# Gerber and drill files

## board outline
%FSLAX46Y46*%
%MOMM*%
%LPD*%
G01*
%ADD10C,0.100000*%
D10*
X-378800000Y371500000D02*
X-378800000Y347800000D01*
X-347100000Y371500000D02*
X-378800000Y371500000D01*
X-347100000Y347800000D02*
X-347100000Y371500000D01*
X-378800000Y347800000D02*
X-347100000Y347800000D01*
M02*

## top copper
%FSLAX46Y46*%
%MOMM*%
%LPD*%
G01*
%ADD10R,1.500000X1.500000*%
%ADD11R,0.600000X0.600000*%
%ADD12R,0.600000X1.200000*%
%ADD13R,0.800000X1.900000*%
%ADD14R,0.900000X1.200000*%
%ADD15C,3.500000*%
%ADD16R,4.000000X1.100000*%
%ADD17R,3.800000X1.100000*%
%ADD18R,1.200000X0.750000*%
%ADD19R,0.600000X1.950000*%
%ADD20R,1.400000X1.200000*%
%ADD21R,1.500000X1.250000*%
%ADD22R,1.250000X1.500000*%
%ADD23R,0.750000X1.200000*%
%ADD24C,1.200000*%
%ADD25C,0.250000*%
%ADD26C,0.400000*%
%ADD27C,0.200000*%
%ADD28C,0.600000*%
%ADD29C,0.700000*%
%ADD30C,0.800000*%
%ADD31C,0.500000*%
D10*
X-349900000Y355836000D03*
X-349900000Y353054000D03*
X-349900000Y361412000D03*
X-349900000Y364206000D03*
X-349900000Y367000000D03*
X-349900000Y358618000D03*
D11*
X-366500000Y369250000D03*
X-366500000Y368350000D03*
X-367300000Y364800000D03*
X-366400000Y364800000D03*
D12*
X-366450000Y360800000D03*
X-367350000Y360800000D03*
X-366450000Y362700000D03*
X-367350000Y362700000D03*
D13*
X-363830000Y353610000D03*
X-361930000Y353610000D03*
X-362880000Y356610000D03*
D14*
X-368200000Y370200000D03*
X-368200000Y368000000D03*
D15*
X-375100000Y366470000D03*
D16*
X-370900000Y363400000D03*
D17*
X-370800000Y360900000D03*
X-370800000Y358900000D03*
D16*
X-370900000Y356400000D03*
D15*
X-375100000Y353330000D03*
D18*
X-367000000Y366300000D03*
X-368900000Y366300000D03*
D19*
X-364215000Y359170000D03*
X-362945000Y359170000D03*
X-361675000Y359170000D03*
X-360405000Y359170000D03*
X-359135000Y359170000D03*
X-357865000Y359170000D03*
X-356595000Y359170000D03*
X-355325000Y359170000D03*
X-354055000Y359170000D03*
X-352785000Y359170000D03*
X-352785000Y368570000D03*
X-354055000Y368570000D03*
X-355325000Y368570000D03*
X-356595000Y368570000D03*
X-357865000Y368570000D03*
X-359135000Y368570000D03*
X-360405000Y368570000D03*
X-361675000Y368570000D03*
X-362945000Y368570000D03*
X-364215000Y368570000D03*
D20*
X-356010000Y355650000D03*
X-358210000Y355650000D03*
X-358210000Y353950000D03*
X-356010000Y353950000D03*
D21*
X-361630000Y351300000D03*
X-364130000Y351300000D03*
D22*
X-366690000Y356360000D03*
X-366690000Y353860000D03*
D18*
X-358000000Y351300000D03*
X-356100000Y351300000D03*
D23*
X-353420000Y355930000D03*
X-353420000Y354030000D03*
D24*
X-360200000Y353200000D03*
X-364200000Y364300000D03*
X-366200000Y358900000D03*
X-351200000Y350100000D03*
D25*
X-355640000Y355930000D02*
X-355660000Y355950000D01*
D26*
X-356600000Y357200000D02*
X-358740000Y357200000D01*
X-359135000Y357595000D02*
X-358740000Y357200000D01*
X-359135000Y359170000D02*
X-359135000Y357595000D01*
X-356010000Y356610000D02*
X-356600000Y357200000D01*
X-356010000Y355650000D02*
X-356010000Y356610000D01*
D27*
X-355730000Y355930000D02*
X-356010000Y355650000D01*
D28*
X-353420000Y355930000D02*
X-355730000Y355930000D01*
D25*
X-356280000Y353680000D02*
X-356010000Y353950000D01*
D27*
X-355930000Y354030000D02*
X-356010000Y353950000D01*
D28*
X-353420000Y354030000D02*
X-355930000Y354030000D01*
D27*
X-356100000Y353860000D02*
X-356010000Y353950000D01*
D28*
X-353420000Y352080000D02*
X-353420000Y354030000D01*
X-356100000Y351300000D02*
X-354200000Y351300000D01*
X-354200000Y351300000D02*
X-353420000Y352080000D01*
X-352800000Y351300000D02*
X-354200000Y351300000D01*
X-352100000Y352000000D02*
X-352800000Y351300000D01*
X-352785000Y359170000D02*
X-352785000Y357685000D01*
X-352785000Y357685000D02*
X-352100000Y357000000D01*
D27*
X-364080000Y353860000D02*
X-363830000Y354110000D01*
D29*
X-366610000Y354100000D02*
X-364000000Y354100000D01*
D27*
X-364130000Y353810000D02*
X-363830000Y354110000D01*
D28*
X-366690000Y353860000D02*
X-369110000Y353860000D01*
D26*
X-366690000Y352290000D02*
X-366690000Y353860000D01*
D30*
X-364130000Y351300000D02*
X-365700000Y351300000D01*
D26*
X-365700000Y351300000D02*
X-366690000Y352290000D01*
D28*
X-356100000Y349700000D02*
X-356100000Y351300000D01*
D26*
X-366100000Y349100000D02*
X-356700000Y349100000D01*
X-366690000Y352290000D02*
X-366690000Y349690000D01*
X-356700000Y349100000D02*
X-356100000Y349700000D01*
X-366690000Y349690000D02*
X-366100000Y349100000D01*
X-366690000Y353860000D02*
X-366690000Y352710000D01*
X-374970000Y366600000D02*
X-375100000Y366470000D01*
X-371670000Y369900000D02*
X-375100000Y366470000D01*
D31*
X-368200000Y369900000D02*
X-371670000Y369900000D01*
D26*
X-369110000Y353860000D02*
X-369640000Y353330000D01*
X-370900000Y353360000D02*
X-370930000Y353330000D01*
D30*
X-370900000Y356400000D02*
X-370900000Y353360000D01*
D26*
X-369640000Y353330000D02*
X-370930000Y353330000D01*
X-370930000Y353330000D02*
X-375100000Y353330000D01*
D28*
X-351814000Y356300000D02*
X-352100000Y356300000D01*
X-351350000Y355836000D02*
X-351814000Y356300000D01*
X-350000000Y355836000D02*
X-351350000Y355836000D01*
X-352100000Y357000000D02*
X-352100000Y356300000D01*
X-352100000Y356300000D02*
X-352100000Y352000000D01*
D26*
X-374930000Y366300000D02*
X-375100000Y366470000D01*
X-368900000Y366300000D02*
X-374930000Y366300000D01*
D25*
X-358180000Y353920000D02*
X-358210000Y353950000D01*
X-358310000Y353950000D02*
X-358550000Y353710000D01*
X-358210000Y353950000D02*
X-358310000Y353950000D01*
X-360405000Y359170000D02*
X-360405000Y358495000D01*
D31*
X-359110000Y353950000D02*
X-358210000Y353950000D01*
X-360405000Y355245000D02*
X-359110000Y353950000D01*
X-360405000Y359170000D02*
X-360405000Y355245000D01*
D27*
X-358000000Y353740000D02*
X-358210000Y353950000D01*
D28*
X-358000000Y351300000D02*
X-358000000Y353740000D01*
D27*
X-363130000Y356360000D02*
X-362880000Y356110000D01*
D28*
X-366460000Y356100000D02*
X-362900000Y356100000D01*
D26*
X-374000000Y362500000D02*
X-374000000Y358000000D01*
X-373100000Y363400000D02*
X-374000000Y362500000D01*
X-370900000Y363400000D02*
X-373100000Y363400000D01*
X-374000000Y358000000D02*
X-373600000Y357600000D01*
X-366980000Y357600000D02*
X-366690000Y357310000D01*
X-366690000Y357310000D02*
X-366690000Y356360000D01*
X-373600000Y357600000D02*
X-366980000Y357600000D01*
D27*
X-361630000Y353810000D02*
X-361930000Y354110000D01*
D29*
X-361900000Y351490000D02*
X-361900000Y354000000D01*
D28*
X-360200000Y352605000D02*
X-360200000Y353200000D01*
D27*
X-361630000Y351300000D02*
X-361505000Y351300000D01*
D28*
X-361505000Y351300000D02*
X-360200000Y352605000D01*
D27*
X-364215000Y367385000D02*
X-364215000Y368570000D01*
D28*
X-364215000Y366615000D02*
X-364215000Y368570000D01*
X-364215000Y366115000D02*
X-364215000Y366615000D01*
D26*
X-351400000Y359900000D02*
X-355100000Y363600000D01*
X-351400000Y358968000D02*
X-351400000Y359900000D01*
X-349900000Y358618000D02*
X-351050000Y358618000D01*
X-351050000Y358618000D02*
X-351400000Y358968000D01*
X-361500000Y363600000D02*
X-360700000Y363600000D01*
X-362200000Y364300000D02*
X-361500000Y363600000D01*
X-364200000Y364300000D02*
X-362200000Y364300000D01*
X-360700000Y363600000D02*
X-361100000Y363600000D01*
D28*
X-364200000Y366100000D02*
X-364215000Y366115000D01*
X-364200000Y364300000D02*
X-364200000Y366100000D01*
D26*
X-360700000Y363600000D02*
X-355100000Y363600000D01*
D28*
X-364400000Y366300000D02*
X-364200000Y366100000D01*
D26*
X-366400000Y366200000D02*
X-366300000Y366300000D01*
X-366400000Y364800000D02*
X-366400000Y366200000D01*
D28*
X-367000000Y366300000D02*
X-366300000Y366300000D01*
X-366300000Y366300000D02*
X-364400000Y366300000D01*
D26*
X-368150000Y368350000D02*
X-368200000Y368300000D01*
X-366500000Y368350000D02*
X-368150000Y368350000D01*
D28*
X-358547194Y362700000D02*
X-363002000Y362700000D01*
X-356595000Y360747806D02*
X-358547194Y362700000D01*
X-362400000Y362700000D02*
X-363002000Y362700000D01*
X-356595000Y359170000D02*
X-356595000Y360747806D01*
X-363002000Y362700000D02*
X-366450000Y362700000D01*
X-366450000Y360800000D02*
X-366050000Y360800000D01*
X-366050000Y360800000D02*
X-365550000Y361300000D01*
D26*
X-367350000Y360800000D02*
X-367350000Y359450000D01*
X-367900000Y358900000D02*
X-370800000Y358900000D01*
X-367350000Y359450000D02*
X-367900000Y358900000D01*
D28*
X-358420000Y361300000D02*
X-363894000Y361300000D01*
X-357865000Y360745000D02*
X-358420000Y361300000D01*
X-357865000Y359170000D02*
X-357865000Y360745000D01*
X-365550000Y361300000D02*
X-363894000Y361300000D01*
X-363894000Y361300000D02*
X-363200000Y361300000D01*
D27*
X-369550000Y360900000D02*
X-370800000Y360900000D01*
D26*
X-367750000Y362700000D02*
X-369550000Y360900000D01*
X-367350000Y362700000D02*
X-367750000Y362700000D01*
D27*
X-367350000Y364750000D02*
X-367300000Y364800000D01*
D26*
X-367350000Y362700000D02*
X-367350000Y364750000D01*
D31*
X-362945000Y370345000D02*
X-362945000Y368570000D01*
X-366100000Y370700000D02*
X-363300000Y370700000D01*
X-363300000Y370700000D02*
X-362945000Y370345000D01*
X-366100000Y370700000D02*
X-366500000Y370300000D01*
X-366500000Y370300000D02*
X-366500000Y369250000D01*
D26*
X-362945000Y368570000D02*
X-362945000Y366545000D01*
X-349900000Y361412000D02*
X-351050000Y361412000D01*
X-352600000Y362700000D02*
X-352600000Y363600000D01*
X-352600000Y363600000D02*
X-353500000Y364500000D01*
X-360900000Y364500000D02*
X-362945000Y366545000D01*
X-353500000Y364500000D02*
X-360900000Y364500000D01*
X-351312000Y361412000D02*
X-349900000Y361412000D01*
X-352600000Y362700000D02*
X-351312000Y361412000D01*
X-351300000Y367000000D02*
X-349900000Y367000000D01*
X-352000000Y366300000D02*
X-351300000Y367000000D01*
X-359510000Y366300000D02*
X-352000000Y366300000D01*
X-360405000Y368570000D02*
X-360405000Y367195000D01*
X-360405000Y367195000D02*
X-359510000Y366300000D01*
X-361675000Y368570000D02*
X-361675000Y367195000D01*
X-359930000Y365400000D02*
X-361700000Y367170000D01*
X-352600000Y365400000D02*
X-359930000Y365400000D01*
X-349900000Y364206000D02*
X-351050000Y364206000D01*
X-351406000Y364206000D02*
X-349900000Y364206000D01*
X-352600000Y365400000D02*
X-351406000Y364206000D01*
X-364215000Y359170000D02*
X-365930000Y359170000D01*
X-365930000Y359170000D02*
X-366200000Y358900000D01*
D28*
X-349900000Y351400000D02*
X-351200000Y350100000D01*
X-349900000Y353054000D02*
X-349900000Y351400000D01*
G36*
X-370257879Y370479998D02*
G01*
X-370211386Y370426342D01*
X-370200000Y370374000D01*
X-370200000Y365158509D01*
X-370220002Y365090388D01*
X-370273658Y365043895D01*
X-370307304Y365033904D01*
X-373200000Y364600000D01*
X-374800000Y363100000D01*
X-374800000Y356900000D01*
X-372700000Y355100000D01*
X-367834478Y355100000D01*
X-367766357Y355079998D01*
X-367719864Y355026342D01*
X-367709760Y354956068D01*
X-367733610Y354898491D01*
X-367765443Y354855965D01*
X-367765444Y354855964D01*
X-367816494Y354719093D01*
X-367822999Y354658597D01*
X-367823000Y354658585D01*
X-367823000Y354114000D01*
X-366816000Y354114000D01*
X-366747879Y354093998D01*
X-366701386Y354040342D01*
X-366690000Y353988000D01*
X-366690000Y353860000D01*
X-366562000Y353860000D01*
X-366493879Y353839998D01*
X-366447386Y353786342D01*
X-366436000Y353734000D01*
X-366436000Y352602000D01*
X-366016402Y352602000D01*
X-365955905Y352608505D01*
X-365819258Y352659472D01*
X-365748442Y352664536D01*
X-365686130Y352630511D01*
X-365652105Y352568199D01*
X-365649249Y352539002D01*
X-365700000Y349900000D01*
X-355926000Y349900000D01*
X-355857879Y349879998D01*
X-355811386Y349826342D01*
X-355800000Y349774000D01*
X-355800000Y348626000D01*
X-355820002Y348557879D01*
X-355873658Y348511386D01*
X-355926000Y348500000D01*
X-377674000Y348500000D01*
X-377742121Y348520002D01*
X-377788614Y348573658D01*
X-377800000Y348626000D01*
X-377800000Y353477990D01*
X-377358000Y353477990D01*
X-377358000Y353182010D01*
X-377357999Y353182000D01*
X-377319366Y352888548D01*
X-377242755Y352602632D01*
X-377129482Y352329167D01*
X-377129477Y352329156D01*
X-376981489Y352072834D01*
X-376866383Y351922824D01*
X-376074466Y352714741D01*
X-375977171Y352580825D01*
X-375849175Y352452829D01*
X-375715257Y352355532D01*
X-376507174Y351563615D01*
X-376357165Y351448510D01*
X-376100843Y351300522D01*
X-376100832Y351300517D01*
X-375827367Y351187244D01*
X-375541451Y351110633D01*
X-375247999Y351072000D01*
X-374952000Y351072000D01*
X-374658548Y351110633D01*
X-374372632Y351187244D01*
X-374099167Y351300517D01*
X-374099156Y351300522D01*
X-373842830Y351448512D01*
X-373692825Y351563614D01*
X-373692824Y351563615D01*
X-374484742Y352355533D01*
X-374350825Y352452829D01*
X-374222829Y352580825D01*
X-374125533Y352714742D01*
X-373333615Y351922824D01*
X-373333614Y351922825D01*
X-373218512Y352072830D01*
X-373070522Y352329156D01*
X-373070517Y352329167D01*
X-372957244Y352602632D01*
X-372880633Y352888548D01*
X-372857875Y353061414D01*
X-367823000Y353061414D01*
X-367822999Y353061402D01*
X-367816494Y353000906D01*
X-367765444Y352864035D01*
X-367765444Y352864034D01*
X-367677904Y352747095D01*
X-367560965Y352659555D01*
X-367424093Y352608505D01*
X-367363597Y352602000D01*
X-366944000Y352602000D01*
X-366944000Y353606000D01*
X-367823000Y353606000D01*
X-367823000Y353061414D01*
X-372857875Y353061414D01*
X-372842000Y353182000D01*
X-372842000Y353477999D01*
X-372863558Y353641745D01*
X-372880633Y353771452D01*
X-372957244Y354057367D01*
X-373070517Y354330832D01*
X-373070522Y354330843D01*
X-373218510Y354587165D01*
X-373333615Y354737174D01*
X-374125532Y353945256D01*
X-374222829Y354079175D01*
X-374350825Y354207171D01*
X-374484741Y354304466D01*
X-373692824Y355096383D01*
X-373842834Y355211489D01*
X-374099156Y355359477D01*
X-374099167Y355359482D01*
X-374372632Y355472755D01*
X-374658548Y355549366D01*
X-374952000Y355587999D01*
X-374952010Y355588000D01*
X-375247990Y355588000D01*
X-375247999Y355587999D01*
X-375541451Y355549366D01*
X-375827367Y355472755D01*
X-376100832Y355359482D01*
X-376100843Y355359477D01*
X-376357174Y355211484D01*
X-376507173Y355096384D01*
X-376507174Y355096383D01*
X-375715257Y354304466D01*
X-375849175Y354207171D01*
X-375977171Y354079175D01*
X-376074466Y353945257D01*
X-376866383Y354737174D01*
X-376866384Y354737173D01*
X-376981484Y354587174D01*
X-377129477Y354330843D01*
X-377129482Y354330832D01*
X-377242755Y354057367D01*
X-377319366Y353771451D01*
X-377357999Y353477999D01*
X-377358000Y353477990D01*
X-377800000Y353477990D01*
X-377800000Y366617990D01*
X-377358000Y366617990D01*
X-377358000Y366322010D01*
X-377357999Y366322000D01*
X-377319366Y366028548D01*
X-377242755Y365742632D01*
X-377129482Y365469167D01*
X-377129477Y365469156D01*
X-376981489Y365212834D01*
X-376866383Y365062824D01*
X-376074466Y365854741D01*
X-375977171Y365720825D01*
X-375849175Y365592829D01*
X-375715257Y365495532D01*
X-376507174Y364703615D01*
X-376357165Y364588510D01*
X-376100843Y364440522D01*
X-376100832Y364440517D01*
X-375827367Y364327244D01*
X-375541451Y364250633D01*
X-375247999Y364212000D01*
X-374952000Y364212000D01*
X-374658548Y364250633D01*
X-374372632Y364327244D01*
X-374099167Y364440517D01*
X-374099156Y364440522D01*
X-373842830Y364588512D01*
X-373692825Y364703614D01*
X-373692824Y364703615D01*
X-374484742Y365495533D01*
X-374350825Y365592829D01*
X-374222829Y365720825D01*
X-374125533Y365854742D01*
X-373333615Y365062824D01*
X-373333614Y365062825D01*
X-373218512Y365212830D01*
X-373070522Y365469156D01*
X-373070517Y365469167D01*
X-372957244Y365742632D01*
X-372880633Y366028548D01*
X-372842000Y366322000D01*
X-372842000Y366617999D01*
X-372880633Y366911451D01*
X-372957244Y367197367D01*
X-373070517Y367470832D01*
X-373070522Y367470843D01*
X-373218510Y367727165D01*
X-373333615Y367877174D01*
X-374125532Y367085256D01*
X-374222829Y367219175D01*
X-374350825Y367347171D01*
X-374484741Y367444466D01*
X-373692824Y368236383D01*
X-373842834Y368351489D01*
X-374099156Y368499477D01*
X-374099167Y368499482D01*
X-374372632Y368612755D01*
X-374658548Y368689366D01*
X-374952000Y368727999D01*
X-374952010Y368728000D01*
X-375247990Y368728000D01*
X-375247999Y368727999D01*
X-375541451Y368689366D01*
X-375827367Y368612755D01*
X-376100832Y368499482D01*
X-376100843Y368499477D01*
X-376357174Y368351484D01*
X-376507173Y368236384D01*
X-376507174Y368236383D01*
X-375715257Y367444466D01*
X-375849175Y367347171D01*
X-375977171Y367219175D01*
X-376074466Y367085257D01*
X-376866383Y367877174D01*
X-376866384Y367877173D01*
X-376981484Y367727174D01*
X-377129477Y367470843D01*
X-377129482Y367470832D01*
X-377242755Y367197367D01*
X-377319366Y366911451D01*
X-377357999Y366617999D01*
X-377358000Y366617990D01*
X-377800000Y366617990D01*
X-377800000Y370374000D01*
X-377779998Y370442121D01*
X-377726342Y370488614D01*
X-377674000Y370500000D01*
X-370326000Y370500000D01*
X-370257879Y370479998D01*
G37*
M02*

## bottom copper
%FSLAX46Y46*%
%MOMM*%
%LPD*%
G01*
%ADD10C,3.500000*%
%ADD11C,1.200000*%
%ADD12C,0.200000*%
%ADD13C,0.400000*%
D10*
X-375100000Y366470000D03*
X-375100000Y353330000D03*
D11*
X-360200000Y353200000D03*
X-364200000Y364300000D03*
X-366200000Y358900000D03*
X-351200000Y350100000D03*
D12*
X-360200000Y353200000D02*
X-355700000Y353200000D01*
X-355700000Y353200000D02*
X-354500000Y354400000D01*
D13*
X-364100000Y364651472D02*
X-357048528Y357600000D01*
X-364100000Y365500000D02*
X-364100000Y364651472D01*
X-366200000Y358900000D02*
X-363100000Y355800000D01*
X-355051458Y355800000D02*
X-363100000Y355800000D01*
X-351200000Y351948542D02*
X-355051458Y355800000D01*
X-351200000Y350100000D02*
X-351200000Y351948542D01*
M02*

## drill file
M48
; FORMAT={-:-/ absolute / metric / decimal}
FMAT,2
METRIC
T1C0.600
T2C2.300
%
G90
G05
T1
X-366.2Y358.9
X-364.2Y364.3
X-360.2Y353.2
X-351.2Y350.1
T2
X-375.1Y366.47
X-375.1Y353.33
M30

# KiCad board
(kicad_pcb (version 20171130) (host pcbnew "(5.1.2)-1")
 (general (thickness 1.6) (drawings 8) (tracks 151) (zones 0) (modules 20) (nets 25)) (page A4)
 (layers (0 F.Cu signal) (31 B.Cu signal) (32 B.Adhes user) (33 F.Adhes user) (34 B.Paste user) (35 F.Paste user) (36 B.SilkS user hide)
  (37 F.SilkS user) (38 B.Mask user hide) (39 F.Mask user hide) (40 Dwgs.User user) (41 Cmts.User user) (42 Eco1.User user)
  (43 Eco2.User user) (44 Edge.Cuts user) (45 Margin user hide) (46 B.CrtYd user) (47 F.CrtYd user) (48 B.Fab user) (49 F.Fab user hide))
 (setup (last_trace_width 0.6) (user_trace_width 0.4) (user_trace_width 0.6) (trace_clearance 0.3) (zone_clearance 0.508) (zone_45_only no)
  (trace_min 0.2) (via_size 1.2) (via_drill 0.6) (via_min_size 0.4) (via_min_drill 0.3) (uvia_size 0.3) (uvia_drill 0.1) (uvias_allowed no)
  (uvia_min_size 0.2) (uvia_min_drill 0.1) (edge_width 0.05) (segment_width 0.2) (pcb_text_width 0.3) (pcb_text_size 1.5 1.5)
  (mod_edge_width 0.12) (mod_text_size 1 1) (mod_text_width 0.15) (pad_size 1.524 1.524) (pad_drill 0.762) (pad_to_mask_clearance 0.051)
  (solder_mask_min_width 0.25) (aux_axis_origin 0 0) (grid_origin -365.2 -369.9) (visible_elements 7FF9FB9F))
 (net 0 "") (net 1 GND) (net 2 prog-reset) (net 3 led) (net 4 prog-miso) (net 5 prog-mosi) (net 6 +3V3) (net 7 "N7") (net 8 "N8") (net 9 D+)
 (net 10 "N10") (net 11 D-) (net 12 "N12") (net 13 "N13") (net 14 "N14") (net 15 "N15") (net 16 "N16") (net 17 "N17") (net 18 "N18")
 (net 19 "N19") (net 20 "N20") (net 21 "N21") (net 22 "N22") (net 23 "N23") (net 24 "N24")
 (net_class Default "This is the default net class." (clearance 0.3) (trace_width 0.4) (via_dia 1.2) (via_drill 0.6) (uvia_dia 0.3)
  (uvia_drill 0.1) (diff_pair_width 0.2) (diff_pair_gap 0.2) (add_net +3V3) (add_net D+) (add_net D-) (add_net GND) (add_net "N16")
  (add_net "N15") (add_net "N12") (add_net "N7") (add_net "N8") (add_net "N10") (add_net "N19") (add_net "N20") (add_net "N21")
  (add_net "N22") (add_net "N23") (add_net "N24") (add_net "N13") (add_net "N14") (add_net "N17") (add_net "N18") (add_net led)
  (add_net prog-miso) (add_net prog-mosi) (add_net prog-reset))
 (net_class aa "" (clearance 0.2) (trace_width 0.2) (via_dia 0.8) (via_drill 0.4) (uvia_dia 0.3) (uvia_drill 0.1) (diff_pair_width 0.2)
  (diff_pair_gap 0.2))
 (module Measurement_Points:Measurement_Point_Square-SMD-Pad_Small (layer F.Cu) (at -349.9 -355.6)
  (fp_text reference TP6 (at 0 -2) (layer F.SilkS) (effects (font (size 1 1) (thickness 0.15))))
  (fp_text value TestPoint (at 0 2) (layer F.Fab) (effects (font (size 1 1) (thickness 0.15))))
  (pad 1 smd rect (at 0 -0.236) (size 1.5 1.5) (layers F.Cu F.Mask) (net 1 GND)))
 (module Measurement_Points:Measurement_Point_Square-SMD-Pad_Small (layer F.Cu) (at -349.9 -352.8)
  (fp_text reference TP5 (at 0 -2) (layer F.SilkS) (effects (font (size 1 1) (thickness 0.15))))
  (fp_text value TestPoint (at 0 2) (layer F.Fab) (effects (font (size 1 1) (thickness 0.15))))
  (pad 1 smd rect (at 0 -0.254) (size 1.5 1.5) (layers F.Cu F.Mask) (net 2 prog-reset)))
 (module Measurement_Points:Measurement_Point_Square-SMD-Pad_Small (layer F.Cu) (at -349.9 -360.65)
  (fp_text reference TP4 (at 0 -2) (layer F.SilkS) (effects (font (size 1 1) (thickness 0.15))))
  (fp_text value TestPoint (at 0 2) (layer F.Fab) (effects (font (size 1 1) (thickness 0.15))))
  (pad 1 smd rect (at 0 -0.762) (size 1.5 1.5) (layers F.Cu F.Mask) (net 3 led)))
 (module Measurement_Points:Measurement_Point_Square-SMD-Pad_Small (layer F.Cu) (at -349.9 -363.1)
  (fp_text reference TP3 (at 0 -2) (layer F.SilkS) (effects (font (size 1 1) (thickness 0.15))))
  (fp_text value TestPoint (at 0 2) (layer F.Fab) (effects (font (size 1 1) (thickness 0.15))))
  (pad 1 smd rect (at 0 -1.106) (size 1.5 1.5) (layers F.Cu F.Mask) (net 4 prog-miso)))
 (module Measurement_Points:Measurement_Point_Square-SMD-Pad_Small (layer F.Cu) (at -349.9 -367)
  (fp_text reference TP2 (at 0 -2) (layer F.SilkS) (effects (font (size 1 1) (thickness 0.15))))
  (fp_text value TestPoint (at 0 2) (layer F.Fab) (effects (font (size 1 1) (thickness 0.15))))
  (pad 1 smd rect (at 0 0) (size 1.5 1.5) (layers F.Cu F.Mask) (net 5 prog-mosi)))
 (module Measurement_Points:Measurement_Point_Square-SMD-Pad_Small (layer F.Cu) (at -349.9 -358.11)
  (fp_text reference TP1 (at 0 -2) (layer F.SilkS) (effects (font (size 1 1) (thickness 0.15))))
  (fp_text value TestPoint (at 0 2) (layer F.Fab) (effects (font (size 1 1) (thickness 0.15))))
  (pad 1 smd rect (at 0 -0.508) (size 1.5 1.5) (layers F.Cu F.Mask) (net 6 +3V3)))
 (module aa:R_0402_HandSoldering (layer F.Cu) (at -366.5 -368.8 270)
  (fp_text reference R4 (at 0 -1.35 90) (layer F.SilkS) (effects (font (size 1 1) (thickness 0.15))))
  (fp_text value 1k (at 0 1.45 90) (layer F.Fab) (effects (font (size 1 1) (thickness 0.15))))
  (pad 1 smd rect (at -0.45 0 270) (size 0.6 0.6) (layers F.Cu F.Paste F.Mask) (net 3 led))
  (pad 2 smd rect (at 0.45 0 270) (size 0.6 0.6) (layers F.Cu F.Paste F.Mask) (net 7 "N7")))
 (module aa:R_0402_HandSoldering (layer F.Cu) (at -366.85 -364.8)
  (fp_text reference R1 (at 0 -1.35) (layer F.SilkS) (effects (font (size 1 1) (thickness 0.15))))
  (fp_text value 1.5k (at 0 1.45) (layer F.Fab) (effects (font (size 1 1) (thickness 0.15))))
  (pad 1 smd rect (at -0.45 0) (size 0.6 0.6) (layers F.Cu F.Paste F.Mask) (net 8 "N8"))
  (pad 2 smd rect (at 0.45 0) (size 0.6 0.6) (layers F.Cu F.Paste F.Mask) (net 6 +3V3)))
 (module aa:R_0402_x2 (layer F.Cu) (at -366.9 -360.8 180)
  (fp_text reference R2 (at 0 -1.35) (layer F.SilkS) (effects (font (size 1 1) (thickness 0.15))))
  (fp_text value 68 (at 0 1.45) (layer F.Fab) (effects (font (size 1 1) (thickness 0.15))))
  (pad 1 smd rect (at -0.45 0 180) (size 0.6 1.2) (layers F.Cu F.Paste F.Mask) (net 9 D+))
  (pad 2 smd rect (at 0.45 0 180) (size 0.6 1.2) (layers F.Cu F.Paste F.Mask) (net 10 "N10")))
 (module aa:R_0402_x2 (layer F.Cu) (at -366.9 -362.7 180)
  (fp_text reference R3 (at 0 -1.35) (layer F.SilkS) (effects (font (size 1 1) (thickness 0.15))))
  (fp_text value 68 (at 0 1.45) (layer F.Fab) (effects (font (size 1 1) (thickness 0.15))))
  (pad 1 smd rect (at -0.45 0 180) (size 0.6 1.2) (layers F.Cu F.Paste F.Mask) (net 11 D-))
  (pad 2 smd rect (at 0.45 0 180) (size 0.6 1.2) (layers F.Cu F.Paste F.Mask) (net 8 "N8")))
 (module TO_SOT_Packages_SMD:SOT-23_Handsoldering (layer F.Cu) (at -362.88 -355.11 90)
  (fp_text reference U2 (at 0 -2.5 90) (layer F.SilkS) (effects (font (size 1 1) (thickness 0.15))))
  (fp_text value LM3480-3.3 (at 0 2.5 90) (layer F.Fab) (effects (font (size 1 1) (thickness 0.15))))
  (pad 1 smd rect (at -1.5 -0.95 90) (size 1.9 0.8) (layers F.Cu F.Paste F.Mask) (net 1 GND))
  (pad 2 smd rect (at -1.5 0.95 90) (size 1.9 0.8) (layers F.Cu F.Paste F.Mask) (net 6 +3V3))
  (pad 3 smd rect (at 1.5 0 90) (size 1.9 0.8) (layers F.Cu F.Paste F.Mask) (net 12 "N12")))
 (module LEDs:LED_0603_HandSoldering (layer F.Cu) (at -368.2 -369.1 270)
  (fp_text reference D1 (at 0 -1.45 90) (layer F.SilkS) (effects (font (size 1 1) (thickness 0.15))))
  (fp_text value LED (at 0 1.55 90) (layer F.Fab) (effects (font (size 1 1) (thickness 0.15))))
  (pad 1 smd rect (at -1.1 0 270) (size 1.2 0.9) (layers F.Cu F.Paste F.Mask) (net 1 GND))
  (pad 2 smd rect (at 1.1 0 270) (size 1.2 0.9) (layers F.Cu F.Paste F.Mask) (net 7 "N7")))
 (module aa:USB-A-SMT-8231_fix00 (layer F.Cu) (at -375.1 -359.9 270)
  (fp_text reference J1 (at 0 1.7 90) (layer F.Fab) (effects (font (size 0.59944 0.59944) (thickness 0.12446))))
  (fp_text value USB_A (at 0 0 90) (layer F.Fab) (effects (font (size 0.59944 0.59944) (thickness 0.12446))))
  (pad 5 thru_hole circle (at -6.57 0) (size 3.5 3.5) (drill 2.3) (layers *.Cu *.Mask) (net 1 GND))
  (pad 1 smd rect (at -3.5 -4.2 270) (size 1.1 4) (layers F.Cu F.Paste F.Mask) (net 12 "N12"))
  (pad 2 smd rect (at -1 -4.3 270) (size 1.1 3.8) (layers F.Cu F.Paste F.Mask) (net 8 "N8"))
  (pad 3 smd rect (at 1 -4.3 270) (size 1.1 3.8) (layers F.Cu F.Paste F.Mask) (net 10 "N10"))
  (pad 4 smd rect (at 3.5 -4.2 270) (size 1.1 4) (layers F.Cu F.Paste F.Mask) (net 1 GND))
  (pad 5 thru_hole circle (at 6.57 0 270) (size 3.5 3.5) (drill 2.3) (layers *.Cu *.Mask) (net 1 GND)))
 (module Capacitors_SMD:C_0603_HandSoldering (layer F.Cu) (at -367.95 -366.3 180)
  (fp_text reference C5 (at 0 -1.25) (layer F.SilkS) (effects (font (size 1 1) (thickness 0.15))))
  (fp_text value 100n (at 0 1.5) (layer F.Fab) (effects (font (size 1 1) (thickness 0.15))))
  (pad 1 smd rect (at -0.95 0 180) (size 1.2 0.75) (layers F.Cu F.Paste F.Mask) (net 6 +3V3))
  (pad 2 smd rect (at 0.95 0 180) (size 1.2 0.75) (layers F.Cu F.Paste F.Mask) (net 1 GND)))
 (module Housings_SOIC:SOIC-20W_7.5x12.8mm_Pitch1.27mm (layer F.Cu) (at -358.5 -363.87 90)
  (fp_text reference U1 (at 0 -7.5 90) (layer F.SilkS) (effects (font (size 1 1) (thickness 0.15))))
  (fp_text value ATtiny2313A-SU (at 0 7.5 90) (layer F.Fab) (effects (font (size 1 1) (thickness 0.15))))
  (pad 1 smd rect (at -4.7 -5.715 90) (size 1.95 0.6) (layers F.Cu F.Paste F.Mask) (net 2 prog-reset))
  (pad 2 smd rect (at -4.7 -4.445 90) (size 1.95 0.6) (layers F.Cu F.Paste F.Mask) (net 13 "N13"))
  (pad 3 smd rect (at -4.7 -3.175 90) (size 1.95 0.6) (layers F.Cu F.Paste F.Mask) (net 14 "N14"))
  (pad 4 smd rect (at -4.7 -1.905 90) (size 1.95 0.6) (layers F.Cu F.Paste F.Mask) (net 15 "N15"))
  (pad 5 smd rect (at -4.7 -0.635 90) (size 1.95 0.6) (layers F.Cu F.Paste F.Mask) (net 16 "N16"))
  (pad 6 smd rect (at -4.7 0.635 90) (size 1.95 0.6) (layers F.Cu F.Paste F.Mask) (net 9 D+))
  (pad 7 smd rect (at -4.7 1.905 90) (size 1.95 0.6) (layers F.Cu F.Paste F.Mask) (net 11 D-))
  (pad 8 smd rect (at -4.7 3.175 90) (size 1.95 0.6) (layers F.Cu F.Paste F.Mask) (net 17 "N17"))
  (pad 9 smd rect (at -4.7 4.445 90) (size 1.95 0.6) (layers F.Cu F.Paste F.Mask) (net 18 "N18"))
  (pad 10 smd rect (at -4.7 5.715 90) (size 1.95 0.6) (layers F.Cu F.Paste F.Mask) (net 1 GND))
  (pad 11 smd rect (at 4.7 5.715 90) (size 1.95 0.6) (layers F.Cu F.Paste F.Mask) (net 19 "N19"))
  (pad 12 smd rect (at 4.7 4.445 90) (size 1.95 0.6) (layers F.Cu F.Paste F.Mask) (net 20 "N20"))
  (pad 13 smd rect (at 4.7 3.175 90) (size 1.95 0.6) (layers F.Cu F.Paste F.Mask) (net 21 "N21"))
  (pad 14 smd rect (at 4.7 1.905 90) (size 1.95 0.6) (layers F.Cu F.Paste F.Mask) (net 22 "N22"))
  (pad 15 smd rect (at 4.7 0.635 90) (size 1.95 0.6) (layers F.Cu F.Paste F.Mask) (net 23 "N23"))
  (pad 16 smd rect (at 4.7 -0.635 90) (size 1.95 0.6) (layers F.Cu F.Paste F.Mask) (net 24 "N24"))
  (pad 17 smd rect (at 4.7 -1.905 90) (size 1.95 0.6) (layers F.Cu F.Paste F.Mask) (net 5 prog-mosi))
  (pad 18 smd rect (at 4.7 -3.175 90) (size 1.95 0.6) (layers F.Cu F.Paste F.Mask) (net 4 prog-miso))
  (pad 19 smd rect (at 4.7 -4.445 90) (size 1.95 0.6) (layers F.Cu F.Paste F.Mask) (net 3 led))
  (pad 20 smd rect (at 4.7 -5.715 90) (size 1.95 0.6) (layers F.Cu F.Paste F.Mask) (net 6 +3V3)))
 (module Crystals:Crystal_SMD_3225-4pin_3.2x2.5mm (layer F.Cu) (at -357.11 -354.8 180)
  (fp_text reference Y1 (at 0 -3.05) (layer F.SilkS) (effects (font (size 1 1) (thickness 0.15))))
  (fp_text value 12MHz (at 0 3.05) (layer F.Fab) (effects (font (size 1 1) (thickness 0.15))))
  (pad 1 smd rect (at -1.1 0.85 180) (size 1.4 1.2) (layers F.Cu F.Paste F.Mask) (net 16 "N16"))
  (pad 2 smd rect (at 1.1 0.85 180) (size 1.4 1.2) (layers F.Cu F.Paste F.Mask) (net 1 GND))
  (pad 3 smd rect (at 1.1 -0.85 180) (size 1.4 1.2) (layers F.Cu F.Paste F.Mask) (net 15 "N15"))
  (pad 4 smd rect (at -1.1 -0.85 180) (size 1.4 1.2) (layers F.Cu F.Paste F.Mask) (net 1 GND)))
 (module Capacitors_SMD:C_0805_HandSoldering (layer F.Cu) (at -362.88 -351.3 180)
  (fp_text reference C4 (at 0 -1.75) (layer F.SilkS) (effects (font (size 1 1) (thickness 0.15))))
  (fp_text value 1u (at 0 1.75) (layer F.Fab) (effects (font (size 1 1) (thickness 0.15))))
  (pad 1 smd rect (at -1.25 0 180) (size 1.5 1.25) (layers F.Cu F.Paste F.Mask) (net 6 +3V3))
  (pad 2 smd rect (at 1.25 0 180) (size 1.5 1.25) (layers F.Cu F.Paste F.Mask) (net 1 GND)))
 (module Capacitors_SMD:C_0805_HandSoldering (layer F.Cu) (at -366.69 -355.11 270)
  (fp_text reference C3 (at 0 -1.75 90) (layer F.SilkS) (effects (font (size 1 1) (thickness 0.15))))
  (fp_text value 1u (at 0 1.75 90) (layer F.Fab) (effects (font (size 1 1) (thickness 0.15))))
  (pad 1 smd rect (at -1.25 0 270) (size 1.5 1.25) (layers F.Cu F.Paste F.Mask) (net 12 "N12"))
  (pad 2 smd rect (at 1.25 0 270) (size 1.5 1.25) (layers F.Cu F.Paste F.Mask) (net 1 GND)))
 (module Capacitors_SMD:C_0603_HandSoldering (layer F.Cu) (at -357.05 -351.3)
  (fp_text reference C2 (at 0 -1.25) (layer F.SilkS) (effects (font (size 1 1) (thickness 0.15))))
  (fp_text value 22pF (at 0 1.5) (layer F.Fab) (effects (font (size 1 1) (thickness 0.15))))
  (pad 1 smd rect (at -0.95 0) (size 1.2 0.75) (layers F.Cu F.Paste F.Mask) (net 15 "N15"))
  (pad 2 smd rect (at 0.95 0) (size 1.2 0.75) (layers F.Cu F.Paste F.Mask) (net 1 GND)))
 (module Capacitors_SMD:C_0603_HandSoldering (layer F.Cu) (at -353.42 -354.98 270)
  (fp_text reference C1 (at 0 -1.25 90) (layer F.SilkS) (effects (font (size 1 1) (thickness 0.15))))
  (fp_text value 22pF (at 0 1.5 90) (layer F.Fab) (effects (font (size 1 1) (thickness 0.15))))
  (pad 1 smd rect (at -0.95 0 270) (size 1.2 0.75) (layers F.Cu F.Paste F.Mask) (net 16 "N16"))
  (pad 2 smd rect (at 0.95 0 270) (size 1.2 0.75) (layers F.Cu F.Paste F.Mask) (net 1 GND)))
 (gr_line (start -378.8 -371.5) (end -378.8 -347.8) (layer Edge.Cuts) (width 0.1))
 (gr_line (start -347.1 -371.5) (end -378.8 -371.5) (layer Edge.Cuts) (width 0.1))
 (gr_line (start -347.1 -347.8) (end -347.1 -371.5) (layer Edge.Cuts) (width 0.1))
 (gr_line (start -378.8 -347.8) (end -347.1 -347.8) (layer Edge.Cuts) (width 0.1))
 (segment (start -355.64 -355.93) (end -355.66 -355.95) (width 0.25) (layer F.Cu) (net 16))
 (segment (start -356.6 -357.2) (end -358.74 -357.2) (width 0.4) (layer F.Cu) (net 16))
 (segment (start -359.135 -357.595) (end -358.74 -357.2) (width 0.4) (layer F.Cu) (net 16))
 (segment (start -359.135 -359.17) (end -359.135 -357.595) (width 0.4) (layer F.Cu) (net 16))
 (segment (start -356.01 -356.61) (end -356.6 -357.2) (width 0.4) (layer F.Cu) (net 16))
 (segment (start -356.01 -355.65) (end -356.01 -356.61) (width 0.4) (layer F.Cu) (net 16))
 (segment (start -355.73 -355.93) (end -356.01 -355.65) (width 0.2) (layer F.Cu) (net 16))
 (segment (start -353.42 -355.93) (end -355.73 -355.93) (width 0.6) (layer F.Cu) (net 16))
 (segment (start -356.28 -353.68) (end -356.01 -353.95) (width 0.25) (layer F.Cu) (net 1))
 (segment (start -355.93 -354.03) (end -356.01 -353.95) (width 0.2) (layer F.Cu) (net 1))
 (segment (start -353.42 -354.03) (end -355.93 -354.03) (width 0.6) (layer F.Cu) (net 1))
 (segment (start -356.1 -353.86) (end -356.01 -353.95) (width 0.2) (layer F.Cu) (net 1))
 (segment (start -353.42 -352.08) (end -353.42 -354.03) (width 0.6) (layer F.Cu) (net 1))
 (segment (start -356.1 -351.3) (end -354.2 -351.3) (width 0.6) (layer F.Cu) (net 1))
 (segment (start -354.2 -351.3) (end -353.42 -352.08) (width 0.6) (layer F.Cu) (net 1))
 (segment (start -352.8 -351.3) (end -354.2 -351.3) (width 0.6) (layer F.Cu) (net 1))
 (segment (start -352.1 -352) (end -352.8 -351.3) (width 0.6) (layer F.Cu) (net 1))
 (segment (start -352.785 -359.17) (end -352.785 -357.685) (width 0.6) (layer F.Cu) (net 1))
 (segment (start -352.785 -357.685) (end -352.1 -357) (width 0.6) (layer F.Cu) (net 1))
 (segment (start -364.08 -353.86) (end -363.83 -354.11) (width 0.2) (layer F.Cu) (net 1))
 (segment (start -366.61 -354.1) (end -364 -354.1) (width 0.7) (layer F.Cu) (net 1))
 (segment (start -364.13 -353.81) (end -363.83 -354.11) (width 0.2) (layer F.Cu) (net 1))
 (segment (start -366.69 -353.86) (end -369.11 -353.86) (width 0.6) (layer F.Cu) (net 1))
 (segment (start -366.69 -352.29) (end -366.69 -353.86) (width 0.4) (layer F.Cu) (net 1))
 (segment (start -364.13 -351.3) (end -365.7 -351.3) (width 0.8) (layer F.Cu) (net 1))
 (segment (start -365.7 -351.3) (end -366.69 -352.29) (width 0.4) (layer F.Cu) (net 1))
 (segment (start -356.1 -349.7) (end -356.1 -351.3) (width 0.6) (layer F.Cu) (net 1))
 (segment (start -366.1 -349.1) (end -356.7 -349.1) (width 0.4) (layer F.Cu) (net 1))
 (segment (start -366.69 -352.29) (end -366.69 -349.69) (width 0.4) (layer F.Cu) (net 1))
 (segment (start -356.7 -349.1) (end -356.1 -349.7) (width 0.4) (layer F.Cu) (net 1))
 (segment (start -366.69 -349.69) (end -366.1 -349.1) (width 0.4) (layer F.Cu) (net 1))
 (segment (start -366.69 -353.86) (end -366.69 -352.71) (width 0.4) (layer F.Cu) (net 1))
 (segment (start -374.97 -366.6) (end -375.1 -366.47) (width 0.4) (layer F.Cu) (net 1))
 (segment (start -371.67 -369.9) (end -375.1 -366.47) (width 0.4) (layer F.Cu) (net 1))
 (segment (start -368.2 -369.9) (end -371.67 -369.9) (width 0.5) (layer F.Cu) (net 1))
 (segment (start -369.11 -353.86) (end -369.64 -353.33) (width 0.4) (layer F.Cu) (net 1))
 (segment (start -370.9 -353.36) (end -370.93 -353.33) (width 0.4) (layer F.Cu) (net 1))
 (segment (start -370.9 -356.4) (end -370.9 -353.36) (width 0.8) (layer F.Cu) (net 1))
 (segment (start -369.64 -353.33) (end -370.93 -353.33) (width 0.4) (layer F.Cu) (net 1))
 (segment (start -370.93 -353.33) (end -375.1 -353.33) (width 0.4) (layer F.Cu) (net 1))
 (segment (start -351.814 -356.3) (end -352.1 -356.3) (width 0.6) (layer F.Cu) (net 1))
 (segment (start -351.35 -355.836) (end -351.814 -356.3) (width 0.6) (layer F.Cu) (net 1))
 (segment (start -350 -355.836) (end -351.35 -355.836) (width 0.6) (layer F.Cu) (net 1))
 (segment (start -352.1 -357) (end -352.1 -356.3) (width 0.6) (layer F.Cu) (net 1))
 (segment (start -352.1 -356.3) (end -352.1 -352) (width 0.6) (layer F.Cu) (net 1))
 (segment (start -374.93 -366.3) (end -375.1 -366.47) (width 0.4) (layer F.Cu) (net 1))
 (segment (start -368.9 -366.3) (end -374.93 -366.3) (width 0.4) (layer F.Cu) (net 1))
 (segment (start -358.18 -353.92) (end -358.21 -353.95) (width 0.25) (layer F.Cu) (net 15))
 (segment (start -358.31 -353.95) (end -358.55 -353.71) (width 0.25) (layer F.Cu) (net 15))
 (segment (start -358.21 -353.95) (end -358.31 -353.95) (width 0.25) (layer F.Cu) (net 15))
 (segment (start -360.405 -359.17) (end -360.405 -358.495) (width 0.25) (layer F.Cu) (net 15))
 (segment (start -359.11 -353.95) (end -358.21 -353.95) (width 0.5) (layer F.Cu) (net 15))
 (segment (start -360.405 -355.245) (end -359.11 -353.95) (width 0.5) (layer F.Cu) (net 15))
 (segment (start -360.405 -359.17) (end -360.405 -355.245) (width 0.5) (layer F.Cu) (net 15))
 (segment (start -358 -353.74) (end -358.21 -353.95) (width 0.2) (layer F.Cu) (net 15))
 (segment (start -358 -351.3) (end -358 -353.74) (width 0.6) (layer F.Cu) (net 15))
 (segment (start -363.13 -356.36) (end -362.88 -356.11) (width 0.2) (layer F.Cu) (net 12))
 (segment (start -366.46 -356.1) (end -362.9 -356.1) (width 0.6) (layer F.Cu) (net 12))
 (segment (start -374 -362.5) (end -374 -358) (width 0.4) (layer F.Cu) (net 12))
 (segment (start -373.1 -363.4) (end -374 -362.5) (width 0.4) (layer F.Cu) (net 12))
 (segment (start -370.9 -363.4) (end -373.1 -363.4) (width 0.4) (layer F.Cu) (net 12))
 (segment (start -374 -358) (end -373.6 -357.6) (width 0.4) (layer F.Cu) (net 12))
 (segment (start -366.98 -357.6) (end -366.69 -357.31) (width 0.4) (layer F.Cu) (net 12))
 (segment (start -366.69 -357.31) (end -366.69 -356.36) (width 0.4) (layer F.Cu) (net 12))
 (segment (start -373.6 -357.6) (end -366.98 -357.6) (width 0.4) (layer F.Cu) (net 12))
 (segment (start -361.63 -353.81) (end -361.93 -354.11) (width 0.2) (layer F.Cu) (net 6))
 (segment (start -361.9 -351.49) (end -361.9 -354) (width 0.7) (layer F.Cu) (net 6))
 (via (at -360.2 -353.2) (size 1.2) (drill 0.6) (layers F.Cu B.Cu) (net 6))
 (segment (start -360.2 -352.605) (end -360.2 -353.2) (width 0.6) (layer F.Cu) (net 6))
 (segment (start -361.63 -351.3) (end -361.505 -351.3) (width 0.2) (layer F.Cu) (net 6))
 (segment (start -361.505 -351.3) (end -360.2 -352.605) (width 0.6) (layer F.Cu) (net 6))
 (segment (start -364.215 -367.385) (end -364.215 -368.57) (width 0.2) (layer F.Cu) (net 6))
 (segment (start -360.2 -353.2) (end -355.7 -353.2) (width 0.2) (layer B.Cu) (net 6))
 (segment (start -355.7 -353.2) (end -354.5 -354.4) (width 0.2) (layer B.Cu) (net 6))
 (segment (start -364.215 -366.615) (end -364.215 -368.57) (width 0.6) (layer F.Cu) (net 6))
 (segment (start -364.215 -366.115) (end -364.215 -366.615) (width 0.6) (layer F.Cu) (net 6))
 (via (at -364.2 -364.3) (size 1.2) (drill 0.6) (layers F.Cu B.Cu) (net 6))
 (segment (start -364.1 -364.651472) (end -357.048528 -357.6) (width 0.4) (layer B.Cu) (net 6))
 (segment (start -364.1 -365.5) (end -364.1 -364.651472) (width 0.4) (layer B.Cu) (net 6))
 (segment (start -351.4 -359.9) (end -355.1 -363.6) (width 0.4) (layer F.Cu) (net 6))
 (segment (start -351.4 -358.968) (end -351.4 -359.9) (width 0.4) (layer F.Cu) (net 6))
 (segment (start -349.9 -358.618) (end -351.05 -358.618) (width 0.4) (layer F.Cu) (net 6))
 (segment (start -351.05 -358.618) (end -351.4 -358.968) (width 0.4) (layer F.Cu) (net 6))
 (segment (start -361.5 -363.6) (end -360.7 -363.6) (width 0.4) (layer F.Cu) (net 6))
 (segment (start -362.2 -364.3) (end -361.5 -363.6) (width 0.4) (layer F.Cu) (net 6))
 (segment (start -364.2 -364.3) (end -362.2 -364.3) (width 0.4) (layer F.Cu) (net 6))
 (segment (start -360.7 -363.6) (end -361.1 -363.6) (width 0.4) (layer F.Cu) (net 6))
 (segment (start -364.2 -366.1) (end -364.215 -366.115) (width 0.6) (layer F.Cu) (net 6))
 (segment (start -364.2 -364.3) (end -364.2 -366.1) (width 0.6) (layer F.Cu) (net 6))
 (segment (start -360.7 -363.6) (end -355.1 -363.6) (width 0.4) (layer F.Cu) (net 6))
 (segment (start -364.4 -366.3) (end -364.2 -366.1) (width 0.6) (layer F.Cu) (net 6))
 (segment (start -366.4 -366.2) (end -366.3 -366.3) (width 0.4) (layer F.Cu) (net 6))
 (segment (start -366.4 -364.8) (end -366.4 -366.2) (width 0.4) (layer F.Cu) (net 6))
 (segment (start -367 -366.3) (end -366.3 -366.3) (width 0.6) (layer F.Cu) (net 6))
 (segment (start -366.3 -366.3) (end -364.4 -366.3) (width 0.6) (layer F.Cu) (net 6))
 (segment (start -368.15 -368.35) (end -368.2 -368.3) (width 0.4) (layer F.Cu) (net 7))
 (segment (start -366.5 -368.35) (end -368.15 -368.35) (width 0.4) (layer F.Cu) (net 7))
 (segment (start -358.547194 -362.7) (end -363.002 -362.7) (width 0.6) (layer F.Cu) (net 11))
 (segment (start -356.595 -360.747806) (end -358.547194 -362.7) (width 0.6) (layer F.Cu) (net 11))
 (segment (start -362.4 -362.7) (end -363.002 -362.7) (width 0.6) (layer F.Cu) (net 11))
 (segment (start -356.595 -359.17) (end -356.595 -360.747806) (width 0.6) (layer F.Cu) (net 11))
 (segment (start -363.002 -362.7) (end -366.45 -362.7) (width 0.6) (layer F.Cu) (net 11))
 (segment (start -366.45 -360.8) (end -366.05 -360.8) (width 0.6) (layer F.Cu) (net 9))
 (segment (start -366.05 -360.8) (end -365.55 -361.3) (width 0.6) (layer F.Cu) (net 9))
 (segment (start -367.35 -360.8) (end -367.35 -359.45) (width 0.4) (layer F.Cu) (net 10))
 (segment (start -367.9 -358.9) (end -370.8 -358.9) (width 0.4) (layer F.Cu) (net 10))
 (segment (start -367.35 -359.45) (end -367.9 -358.9) (width 0.4) (layer F.Cu) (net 10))
 (segment (start -358.42 -361.3) (end -363.894 -361.3) (width 0.6) (layer F.Cu) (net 9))
 (segment (start -357.865 -360.745) (end -358.42 -361.3) (width 0.6) (layer F.Cu) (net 9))
 (segment (start -357.865 -359.17) (end -357.865 -360.745) (width 0.6) (layer F.Cu) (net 9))
 (segment (start -365.55 -361.3) (end -363.894 -361.3) (width 0.6) (layer F.Cu) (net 9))
 (segment (start -363.894 -361.3) (end -363.2 -361.3) (width 0.6) (layer F.Cu) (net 9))
 (segment (start -369.55 -360.9) (end -370.8 -360.9) (width 0.2) (layer F.Cu) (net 8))
 (segment (start -367.75 -362.7) (end -369.55 -360.9) (width 0.4) (layer F.Cu) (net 8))
 (segment (start -367.35 -362.7) (end -367.75 -362.7) (width 0.4) (layer F.Cu) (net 8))
 (segment (start -367.35 -364.75) (end -367.3 -364.8) (width 0.2) (layer F.Cu) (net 8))
 (segment (start -367.35 -362.7) (end -367.35 -364.75) (width 0.4) (layer F.Cu) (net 8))
 (segment (start -362.945 -370.345) (end -362.945 -368.57) (width 0.5) (layer F.Cu) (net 3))
 (segment (start -366.1 -370.7) (end -363.3 -370.7) (width 0.5) (layer F.Cu) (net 3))
 (segment (start -363.3 -370.7) (end -362.945 -370.345) (width 0.5) (layer F.Cu) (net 3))
 (segment (start -366.1 -370.7) (end -366.5 -370.3) (width 0.5) (layer F.Cu) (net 3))
 (segment (start -366.5 -370.3) (end -366.5 -369.25) (width 0.5) (layer F.Cu) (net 3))
 (segment (start -362.945 -368.57) (end -362.945 -366.545) (width 0.4) (layer F.Cu) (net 3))
 (segment (start -349.9 -361.412) (end -351.05 -361.412) (width 0.4) (layer F.Cu) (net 3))
 (segment (start -352.6 -362.7) (end -352.6 -363.6) (width 0.4) (layer F.Cu) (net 3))
 (segment (start -352.6 -363.6) (end -353.5 -364.5) (width 0.4) (layer F.Cu) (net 3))
 (segment (start -360.9 -364.5) (end -362.945 -366.545) (width 0.4) (layer F.Cu) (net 3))
 (segment (start -353.5 -364.5) (end -360.9 -364.5) (width 0.4) (layer F.Cu) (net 3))
 (segment (start -351.312 -361.412) (end -349.9 -361.412) (width 0.4) (layer F.Cu) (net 3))
 (segment (start -352.6 -362.7) (end -351.312 -361.412) (width 0.4) (layer F.Cu) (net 3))
 (segment (start -351.3 -367) (end -349.9 -367) (width 0.4) (layer F.Cu) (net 5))
 (segment (start -352 -366.3) (end -351.3 -367) (width 0.4) (layer F.Cu) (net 5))
 (segment (start -359.51 -366.3) (end -352 -366.3) (width 0.4) (layer F.Cu) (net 5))
 (segment (start -360.405 -368.57) (end -360.405 -367.195) (width 0.4) (layer F.Cu) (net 5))
 (segment (start -360.405 -367.195) (end -359.51 -366.3) (width 0.4) (layer F.Cu) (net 5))
 (segment (start -361.675 -368.57) (end -361.675 -367.195) (width 0.4) (layer F.Cu) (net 4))
 (segment (start -359.93 -365.4) (end -361.7 -367.17) (width 0.4) (layer F.Cu) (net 4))
 (segment (start -352.6 -365.4) (end -359.93 -365.4) (width 0.4) (layer F.Cu) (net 4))
 (segment (start -349.9 -364.206) (end -351.05 -364.206) (width 0.4) (layer F.Cu) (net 4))
 (segment (start -351.406 -364.206) (end -349.9 -364.206) (width 0.4) (layer F.Cu) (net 4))
 (segment (start -352.6 -365.4) (end -351.406 -364.206) (width 0.4) (layer F.Cu) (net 4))
 (via (at -366.2 -358.9) (size 1.2) (drill 0.6) (layers F.Cu B.Cu) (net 2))
 (segment (start -364.215 -359.17) (end -365.93 -359.17) (width 0.4) (layer F.Cu) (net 2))
 (segment (start -365.93 -359.17) (end -366.2 -358.9) (width 0.4) (layer F.Cu) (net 2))
 (segment (start -366.2 -358.9) (end -363.1 -355.8) (width 0.4) (layer B.Cu) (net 2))
 (via (at -351.2 -350.1) (size 1.2) (drill 0.6) (layers F.Cu B.Cu) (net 2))
 (segment (start -355.051458 -355.8) (end -363.1 -355.8) (width 0.4) (layer B.Cu) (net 2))
 (segment (start -351.2 -351.948542) (end -355.051458 -355.8) (width 0.4) (layer B.Cu) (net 2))
 (segment (start -351.2 -350.1) (end -351.2 -351.948542) (width 0.4) (layer B.Cu) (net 2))
 (segment (start -349.9 -351.4) (end -351.2 -350.1) (width 0.6) (layer F.Cu) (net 2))
 (segment (start -349.9 -353.054) (end -349.9 -351.4) (width 0.6) (layer F.Cu) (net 2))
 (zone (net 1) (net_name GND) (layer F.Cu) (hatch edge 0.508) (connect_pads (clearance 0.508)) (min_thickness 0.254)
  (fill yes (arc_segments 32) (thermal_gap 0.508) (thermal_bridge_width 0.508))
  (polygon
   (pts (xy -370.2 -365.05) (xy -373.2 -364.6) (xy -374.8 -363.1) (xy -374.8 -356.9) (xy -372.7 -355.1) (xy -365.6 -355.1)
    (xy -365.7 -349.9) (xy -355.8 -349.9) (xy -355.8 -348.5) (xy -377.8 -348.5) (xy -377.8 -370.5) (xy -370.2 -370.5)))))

